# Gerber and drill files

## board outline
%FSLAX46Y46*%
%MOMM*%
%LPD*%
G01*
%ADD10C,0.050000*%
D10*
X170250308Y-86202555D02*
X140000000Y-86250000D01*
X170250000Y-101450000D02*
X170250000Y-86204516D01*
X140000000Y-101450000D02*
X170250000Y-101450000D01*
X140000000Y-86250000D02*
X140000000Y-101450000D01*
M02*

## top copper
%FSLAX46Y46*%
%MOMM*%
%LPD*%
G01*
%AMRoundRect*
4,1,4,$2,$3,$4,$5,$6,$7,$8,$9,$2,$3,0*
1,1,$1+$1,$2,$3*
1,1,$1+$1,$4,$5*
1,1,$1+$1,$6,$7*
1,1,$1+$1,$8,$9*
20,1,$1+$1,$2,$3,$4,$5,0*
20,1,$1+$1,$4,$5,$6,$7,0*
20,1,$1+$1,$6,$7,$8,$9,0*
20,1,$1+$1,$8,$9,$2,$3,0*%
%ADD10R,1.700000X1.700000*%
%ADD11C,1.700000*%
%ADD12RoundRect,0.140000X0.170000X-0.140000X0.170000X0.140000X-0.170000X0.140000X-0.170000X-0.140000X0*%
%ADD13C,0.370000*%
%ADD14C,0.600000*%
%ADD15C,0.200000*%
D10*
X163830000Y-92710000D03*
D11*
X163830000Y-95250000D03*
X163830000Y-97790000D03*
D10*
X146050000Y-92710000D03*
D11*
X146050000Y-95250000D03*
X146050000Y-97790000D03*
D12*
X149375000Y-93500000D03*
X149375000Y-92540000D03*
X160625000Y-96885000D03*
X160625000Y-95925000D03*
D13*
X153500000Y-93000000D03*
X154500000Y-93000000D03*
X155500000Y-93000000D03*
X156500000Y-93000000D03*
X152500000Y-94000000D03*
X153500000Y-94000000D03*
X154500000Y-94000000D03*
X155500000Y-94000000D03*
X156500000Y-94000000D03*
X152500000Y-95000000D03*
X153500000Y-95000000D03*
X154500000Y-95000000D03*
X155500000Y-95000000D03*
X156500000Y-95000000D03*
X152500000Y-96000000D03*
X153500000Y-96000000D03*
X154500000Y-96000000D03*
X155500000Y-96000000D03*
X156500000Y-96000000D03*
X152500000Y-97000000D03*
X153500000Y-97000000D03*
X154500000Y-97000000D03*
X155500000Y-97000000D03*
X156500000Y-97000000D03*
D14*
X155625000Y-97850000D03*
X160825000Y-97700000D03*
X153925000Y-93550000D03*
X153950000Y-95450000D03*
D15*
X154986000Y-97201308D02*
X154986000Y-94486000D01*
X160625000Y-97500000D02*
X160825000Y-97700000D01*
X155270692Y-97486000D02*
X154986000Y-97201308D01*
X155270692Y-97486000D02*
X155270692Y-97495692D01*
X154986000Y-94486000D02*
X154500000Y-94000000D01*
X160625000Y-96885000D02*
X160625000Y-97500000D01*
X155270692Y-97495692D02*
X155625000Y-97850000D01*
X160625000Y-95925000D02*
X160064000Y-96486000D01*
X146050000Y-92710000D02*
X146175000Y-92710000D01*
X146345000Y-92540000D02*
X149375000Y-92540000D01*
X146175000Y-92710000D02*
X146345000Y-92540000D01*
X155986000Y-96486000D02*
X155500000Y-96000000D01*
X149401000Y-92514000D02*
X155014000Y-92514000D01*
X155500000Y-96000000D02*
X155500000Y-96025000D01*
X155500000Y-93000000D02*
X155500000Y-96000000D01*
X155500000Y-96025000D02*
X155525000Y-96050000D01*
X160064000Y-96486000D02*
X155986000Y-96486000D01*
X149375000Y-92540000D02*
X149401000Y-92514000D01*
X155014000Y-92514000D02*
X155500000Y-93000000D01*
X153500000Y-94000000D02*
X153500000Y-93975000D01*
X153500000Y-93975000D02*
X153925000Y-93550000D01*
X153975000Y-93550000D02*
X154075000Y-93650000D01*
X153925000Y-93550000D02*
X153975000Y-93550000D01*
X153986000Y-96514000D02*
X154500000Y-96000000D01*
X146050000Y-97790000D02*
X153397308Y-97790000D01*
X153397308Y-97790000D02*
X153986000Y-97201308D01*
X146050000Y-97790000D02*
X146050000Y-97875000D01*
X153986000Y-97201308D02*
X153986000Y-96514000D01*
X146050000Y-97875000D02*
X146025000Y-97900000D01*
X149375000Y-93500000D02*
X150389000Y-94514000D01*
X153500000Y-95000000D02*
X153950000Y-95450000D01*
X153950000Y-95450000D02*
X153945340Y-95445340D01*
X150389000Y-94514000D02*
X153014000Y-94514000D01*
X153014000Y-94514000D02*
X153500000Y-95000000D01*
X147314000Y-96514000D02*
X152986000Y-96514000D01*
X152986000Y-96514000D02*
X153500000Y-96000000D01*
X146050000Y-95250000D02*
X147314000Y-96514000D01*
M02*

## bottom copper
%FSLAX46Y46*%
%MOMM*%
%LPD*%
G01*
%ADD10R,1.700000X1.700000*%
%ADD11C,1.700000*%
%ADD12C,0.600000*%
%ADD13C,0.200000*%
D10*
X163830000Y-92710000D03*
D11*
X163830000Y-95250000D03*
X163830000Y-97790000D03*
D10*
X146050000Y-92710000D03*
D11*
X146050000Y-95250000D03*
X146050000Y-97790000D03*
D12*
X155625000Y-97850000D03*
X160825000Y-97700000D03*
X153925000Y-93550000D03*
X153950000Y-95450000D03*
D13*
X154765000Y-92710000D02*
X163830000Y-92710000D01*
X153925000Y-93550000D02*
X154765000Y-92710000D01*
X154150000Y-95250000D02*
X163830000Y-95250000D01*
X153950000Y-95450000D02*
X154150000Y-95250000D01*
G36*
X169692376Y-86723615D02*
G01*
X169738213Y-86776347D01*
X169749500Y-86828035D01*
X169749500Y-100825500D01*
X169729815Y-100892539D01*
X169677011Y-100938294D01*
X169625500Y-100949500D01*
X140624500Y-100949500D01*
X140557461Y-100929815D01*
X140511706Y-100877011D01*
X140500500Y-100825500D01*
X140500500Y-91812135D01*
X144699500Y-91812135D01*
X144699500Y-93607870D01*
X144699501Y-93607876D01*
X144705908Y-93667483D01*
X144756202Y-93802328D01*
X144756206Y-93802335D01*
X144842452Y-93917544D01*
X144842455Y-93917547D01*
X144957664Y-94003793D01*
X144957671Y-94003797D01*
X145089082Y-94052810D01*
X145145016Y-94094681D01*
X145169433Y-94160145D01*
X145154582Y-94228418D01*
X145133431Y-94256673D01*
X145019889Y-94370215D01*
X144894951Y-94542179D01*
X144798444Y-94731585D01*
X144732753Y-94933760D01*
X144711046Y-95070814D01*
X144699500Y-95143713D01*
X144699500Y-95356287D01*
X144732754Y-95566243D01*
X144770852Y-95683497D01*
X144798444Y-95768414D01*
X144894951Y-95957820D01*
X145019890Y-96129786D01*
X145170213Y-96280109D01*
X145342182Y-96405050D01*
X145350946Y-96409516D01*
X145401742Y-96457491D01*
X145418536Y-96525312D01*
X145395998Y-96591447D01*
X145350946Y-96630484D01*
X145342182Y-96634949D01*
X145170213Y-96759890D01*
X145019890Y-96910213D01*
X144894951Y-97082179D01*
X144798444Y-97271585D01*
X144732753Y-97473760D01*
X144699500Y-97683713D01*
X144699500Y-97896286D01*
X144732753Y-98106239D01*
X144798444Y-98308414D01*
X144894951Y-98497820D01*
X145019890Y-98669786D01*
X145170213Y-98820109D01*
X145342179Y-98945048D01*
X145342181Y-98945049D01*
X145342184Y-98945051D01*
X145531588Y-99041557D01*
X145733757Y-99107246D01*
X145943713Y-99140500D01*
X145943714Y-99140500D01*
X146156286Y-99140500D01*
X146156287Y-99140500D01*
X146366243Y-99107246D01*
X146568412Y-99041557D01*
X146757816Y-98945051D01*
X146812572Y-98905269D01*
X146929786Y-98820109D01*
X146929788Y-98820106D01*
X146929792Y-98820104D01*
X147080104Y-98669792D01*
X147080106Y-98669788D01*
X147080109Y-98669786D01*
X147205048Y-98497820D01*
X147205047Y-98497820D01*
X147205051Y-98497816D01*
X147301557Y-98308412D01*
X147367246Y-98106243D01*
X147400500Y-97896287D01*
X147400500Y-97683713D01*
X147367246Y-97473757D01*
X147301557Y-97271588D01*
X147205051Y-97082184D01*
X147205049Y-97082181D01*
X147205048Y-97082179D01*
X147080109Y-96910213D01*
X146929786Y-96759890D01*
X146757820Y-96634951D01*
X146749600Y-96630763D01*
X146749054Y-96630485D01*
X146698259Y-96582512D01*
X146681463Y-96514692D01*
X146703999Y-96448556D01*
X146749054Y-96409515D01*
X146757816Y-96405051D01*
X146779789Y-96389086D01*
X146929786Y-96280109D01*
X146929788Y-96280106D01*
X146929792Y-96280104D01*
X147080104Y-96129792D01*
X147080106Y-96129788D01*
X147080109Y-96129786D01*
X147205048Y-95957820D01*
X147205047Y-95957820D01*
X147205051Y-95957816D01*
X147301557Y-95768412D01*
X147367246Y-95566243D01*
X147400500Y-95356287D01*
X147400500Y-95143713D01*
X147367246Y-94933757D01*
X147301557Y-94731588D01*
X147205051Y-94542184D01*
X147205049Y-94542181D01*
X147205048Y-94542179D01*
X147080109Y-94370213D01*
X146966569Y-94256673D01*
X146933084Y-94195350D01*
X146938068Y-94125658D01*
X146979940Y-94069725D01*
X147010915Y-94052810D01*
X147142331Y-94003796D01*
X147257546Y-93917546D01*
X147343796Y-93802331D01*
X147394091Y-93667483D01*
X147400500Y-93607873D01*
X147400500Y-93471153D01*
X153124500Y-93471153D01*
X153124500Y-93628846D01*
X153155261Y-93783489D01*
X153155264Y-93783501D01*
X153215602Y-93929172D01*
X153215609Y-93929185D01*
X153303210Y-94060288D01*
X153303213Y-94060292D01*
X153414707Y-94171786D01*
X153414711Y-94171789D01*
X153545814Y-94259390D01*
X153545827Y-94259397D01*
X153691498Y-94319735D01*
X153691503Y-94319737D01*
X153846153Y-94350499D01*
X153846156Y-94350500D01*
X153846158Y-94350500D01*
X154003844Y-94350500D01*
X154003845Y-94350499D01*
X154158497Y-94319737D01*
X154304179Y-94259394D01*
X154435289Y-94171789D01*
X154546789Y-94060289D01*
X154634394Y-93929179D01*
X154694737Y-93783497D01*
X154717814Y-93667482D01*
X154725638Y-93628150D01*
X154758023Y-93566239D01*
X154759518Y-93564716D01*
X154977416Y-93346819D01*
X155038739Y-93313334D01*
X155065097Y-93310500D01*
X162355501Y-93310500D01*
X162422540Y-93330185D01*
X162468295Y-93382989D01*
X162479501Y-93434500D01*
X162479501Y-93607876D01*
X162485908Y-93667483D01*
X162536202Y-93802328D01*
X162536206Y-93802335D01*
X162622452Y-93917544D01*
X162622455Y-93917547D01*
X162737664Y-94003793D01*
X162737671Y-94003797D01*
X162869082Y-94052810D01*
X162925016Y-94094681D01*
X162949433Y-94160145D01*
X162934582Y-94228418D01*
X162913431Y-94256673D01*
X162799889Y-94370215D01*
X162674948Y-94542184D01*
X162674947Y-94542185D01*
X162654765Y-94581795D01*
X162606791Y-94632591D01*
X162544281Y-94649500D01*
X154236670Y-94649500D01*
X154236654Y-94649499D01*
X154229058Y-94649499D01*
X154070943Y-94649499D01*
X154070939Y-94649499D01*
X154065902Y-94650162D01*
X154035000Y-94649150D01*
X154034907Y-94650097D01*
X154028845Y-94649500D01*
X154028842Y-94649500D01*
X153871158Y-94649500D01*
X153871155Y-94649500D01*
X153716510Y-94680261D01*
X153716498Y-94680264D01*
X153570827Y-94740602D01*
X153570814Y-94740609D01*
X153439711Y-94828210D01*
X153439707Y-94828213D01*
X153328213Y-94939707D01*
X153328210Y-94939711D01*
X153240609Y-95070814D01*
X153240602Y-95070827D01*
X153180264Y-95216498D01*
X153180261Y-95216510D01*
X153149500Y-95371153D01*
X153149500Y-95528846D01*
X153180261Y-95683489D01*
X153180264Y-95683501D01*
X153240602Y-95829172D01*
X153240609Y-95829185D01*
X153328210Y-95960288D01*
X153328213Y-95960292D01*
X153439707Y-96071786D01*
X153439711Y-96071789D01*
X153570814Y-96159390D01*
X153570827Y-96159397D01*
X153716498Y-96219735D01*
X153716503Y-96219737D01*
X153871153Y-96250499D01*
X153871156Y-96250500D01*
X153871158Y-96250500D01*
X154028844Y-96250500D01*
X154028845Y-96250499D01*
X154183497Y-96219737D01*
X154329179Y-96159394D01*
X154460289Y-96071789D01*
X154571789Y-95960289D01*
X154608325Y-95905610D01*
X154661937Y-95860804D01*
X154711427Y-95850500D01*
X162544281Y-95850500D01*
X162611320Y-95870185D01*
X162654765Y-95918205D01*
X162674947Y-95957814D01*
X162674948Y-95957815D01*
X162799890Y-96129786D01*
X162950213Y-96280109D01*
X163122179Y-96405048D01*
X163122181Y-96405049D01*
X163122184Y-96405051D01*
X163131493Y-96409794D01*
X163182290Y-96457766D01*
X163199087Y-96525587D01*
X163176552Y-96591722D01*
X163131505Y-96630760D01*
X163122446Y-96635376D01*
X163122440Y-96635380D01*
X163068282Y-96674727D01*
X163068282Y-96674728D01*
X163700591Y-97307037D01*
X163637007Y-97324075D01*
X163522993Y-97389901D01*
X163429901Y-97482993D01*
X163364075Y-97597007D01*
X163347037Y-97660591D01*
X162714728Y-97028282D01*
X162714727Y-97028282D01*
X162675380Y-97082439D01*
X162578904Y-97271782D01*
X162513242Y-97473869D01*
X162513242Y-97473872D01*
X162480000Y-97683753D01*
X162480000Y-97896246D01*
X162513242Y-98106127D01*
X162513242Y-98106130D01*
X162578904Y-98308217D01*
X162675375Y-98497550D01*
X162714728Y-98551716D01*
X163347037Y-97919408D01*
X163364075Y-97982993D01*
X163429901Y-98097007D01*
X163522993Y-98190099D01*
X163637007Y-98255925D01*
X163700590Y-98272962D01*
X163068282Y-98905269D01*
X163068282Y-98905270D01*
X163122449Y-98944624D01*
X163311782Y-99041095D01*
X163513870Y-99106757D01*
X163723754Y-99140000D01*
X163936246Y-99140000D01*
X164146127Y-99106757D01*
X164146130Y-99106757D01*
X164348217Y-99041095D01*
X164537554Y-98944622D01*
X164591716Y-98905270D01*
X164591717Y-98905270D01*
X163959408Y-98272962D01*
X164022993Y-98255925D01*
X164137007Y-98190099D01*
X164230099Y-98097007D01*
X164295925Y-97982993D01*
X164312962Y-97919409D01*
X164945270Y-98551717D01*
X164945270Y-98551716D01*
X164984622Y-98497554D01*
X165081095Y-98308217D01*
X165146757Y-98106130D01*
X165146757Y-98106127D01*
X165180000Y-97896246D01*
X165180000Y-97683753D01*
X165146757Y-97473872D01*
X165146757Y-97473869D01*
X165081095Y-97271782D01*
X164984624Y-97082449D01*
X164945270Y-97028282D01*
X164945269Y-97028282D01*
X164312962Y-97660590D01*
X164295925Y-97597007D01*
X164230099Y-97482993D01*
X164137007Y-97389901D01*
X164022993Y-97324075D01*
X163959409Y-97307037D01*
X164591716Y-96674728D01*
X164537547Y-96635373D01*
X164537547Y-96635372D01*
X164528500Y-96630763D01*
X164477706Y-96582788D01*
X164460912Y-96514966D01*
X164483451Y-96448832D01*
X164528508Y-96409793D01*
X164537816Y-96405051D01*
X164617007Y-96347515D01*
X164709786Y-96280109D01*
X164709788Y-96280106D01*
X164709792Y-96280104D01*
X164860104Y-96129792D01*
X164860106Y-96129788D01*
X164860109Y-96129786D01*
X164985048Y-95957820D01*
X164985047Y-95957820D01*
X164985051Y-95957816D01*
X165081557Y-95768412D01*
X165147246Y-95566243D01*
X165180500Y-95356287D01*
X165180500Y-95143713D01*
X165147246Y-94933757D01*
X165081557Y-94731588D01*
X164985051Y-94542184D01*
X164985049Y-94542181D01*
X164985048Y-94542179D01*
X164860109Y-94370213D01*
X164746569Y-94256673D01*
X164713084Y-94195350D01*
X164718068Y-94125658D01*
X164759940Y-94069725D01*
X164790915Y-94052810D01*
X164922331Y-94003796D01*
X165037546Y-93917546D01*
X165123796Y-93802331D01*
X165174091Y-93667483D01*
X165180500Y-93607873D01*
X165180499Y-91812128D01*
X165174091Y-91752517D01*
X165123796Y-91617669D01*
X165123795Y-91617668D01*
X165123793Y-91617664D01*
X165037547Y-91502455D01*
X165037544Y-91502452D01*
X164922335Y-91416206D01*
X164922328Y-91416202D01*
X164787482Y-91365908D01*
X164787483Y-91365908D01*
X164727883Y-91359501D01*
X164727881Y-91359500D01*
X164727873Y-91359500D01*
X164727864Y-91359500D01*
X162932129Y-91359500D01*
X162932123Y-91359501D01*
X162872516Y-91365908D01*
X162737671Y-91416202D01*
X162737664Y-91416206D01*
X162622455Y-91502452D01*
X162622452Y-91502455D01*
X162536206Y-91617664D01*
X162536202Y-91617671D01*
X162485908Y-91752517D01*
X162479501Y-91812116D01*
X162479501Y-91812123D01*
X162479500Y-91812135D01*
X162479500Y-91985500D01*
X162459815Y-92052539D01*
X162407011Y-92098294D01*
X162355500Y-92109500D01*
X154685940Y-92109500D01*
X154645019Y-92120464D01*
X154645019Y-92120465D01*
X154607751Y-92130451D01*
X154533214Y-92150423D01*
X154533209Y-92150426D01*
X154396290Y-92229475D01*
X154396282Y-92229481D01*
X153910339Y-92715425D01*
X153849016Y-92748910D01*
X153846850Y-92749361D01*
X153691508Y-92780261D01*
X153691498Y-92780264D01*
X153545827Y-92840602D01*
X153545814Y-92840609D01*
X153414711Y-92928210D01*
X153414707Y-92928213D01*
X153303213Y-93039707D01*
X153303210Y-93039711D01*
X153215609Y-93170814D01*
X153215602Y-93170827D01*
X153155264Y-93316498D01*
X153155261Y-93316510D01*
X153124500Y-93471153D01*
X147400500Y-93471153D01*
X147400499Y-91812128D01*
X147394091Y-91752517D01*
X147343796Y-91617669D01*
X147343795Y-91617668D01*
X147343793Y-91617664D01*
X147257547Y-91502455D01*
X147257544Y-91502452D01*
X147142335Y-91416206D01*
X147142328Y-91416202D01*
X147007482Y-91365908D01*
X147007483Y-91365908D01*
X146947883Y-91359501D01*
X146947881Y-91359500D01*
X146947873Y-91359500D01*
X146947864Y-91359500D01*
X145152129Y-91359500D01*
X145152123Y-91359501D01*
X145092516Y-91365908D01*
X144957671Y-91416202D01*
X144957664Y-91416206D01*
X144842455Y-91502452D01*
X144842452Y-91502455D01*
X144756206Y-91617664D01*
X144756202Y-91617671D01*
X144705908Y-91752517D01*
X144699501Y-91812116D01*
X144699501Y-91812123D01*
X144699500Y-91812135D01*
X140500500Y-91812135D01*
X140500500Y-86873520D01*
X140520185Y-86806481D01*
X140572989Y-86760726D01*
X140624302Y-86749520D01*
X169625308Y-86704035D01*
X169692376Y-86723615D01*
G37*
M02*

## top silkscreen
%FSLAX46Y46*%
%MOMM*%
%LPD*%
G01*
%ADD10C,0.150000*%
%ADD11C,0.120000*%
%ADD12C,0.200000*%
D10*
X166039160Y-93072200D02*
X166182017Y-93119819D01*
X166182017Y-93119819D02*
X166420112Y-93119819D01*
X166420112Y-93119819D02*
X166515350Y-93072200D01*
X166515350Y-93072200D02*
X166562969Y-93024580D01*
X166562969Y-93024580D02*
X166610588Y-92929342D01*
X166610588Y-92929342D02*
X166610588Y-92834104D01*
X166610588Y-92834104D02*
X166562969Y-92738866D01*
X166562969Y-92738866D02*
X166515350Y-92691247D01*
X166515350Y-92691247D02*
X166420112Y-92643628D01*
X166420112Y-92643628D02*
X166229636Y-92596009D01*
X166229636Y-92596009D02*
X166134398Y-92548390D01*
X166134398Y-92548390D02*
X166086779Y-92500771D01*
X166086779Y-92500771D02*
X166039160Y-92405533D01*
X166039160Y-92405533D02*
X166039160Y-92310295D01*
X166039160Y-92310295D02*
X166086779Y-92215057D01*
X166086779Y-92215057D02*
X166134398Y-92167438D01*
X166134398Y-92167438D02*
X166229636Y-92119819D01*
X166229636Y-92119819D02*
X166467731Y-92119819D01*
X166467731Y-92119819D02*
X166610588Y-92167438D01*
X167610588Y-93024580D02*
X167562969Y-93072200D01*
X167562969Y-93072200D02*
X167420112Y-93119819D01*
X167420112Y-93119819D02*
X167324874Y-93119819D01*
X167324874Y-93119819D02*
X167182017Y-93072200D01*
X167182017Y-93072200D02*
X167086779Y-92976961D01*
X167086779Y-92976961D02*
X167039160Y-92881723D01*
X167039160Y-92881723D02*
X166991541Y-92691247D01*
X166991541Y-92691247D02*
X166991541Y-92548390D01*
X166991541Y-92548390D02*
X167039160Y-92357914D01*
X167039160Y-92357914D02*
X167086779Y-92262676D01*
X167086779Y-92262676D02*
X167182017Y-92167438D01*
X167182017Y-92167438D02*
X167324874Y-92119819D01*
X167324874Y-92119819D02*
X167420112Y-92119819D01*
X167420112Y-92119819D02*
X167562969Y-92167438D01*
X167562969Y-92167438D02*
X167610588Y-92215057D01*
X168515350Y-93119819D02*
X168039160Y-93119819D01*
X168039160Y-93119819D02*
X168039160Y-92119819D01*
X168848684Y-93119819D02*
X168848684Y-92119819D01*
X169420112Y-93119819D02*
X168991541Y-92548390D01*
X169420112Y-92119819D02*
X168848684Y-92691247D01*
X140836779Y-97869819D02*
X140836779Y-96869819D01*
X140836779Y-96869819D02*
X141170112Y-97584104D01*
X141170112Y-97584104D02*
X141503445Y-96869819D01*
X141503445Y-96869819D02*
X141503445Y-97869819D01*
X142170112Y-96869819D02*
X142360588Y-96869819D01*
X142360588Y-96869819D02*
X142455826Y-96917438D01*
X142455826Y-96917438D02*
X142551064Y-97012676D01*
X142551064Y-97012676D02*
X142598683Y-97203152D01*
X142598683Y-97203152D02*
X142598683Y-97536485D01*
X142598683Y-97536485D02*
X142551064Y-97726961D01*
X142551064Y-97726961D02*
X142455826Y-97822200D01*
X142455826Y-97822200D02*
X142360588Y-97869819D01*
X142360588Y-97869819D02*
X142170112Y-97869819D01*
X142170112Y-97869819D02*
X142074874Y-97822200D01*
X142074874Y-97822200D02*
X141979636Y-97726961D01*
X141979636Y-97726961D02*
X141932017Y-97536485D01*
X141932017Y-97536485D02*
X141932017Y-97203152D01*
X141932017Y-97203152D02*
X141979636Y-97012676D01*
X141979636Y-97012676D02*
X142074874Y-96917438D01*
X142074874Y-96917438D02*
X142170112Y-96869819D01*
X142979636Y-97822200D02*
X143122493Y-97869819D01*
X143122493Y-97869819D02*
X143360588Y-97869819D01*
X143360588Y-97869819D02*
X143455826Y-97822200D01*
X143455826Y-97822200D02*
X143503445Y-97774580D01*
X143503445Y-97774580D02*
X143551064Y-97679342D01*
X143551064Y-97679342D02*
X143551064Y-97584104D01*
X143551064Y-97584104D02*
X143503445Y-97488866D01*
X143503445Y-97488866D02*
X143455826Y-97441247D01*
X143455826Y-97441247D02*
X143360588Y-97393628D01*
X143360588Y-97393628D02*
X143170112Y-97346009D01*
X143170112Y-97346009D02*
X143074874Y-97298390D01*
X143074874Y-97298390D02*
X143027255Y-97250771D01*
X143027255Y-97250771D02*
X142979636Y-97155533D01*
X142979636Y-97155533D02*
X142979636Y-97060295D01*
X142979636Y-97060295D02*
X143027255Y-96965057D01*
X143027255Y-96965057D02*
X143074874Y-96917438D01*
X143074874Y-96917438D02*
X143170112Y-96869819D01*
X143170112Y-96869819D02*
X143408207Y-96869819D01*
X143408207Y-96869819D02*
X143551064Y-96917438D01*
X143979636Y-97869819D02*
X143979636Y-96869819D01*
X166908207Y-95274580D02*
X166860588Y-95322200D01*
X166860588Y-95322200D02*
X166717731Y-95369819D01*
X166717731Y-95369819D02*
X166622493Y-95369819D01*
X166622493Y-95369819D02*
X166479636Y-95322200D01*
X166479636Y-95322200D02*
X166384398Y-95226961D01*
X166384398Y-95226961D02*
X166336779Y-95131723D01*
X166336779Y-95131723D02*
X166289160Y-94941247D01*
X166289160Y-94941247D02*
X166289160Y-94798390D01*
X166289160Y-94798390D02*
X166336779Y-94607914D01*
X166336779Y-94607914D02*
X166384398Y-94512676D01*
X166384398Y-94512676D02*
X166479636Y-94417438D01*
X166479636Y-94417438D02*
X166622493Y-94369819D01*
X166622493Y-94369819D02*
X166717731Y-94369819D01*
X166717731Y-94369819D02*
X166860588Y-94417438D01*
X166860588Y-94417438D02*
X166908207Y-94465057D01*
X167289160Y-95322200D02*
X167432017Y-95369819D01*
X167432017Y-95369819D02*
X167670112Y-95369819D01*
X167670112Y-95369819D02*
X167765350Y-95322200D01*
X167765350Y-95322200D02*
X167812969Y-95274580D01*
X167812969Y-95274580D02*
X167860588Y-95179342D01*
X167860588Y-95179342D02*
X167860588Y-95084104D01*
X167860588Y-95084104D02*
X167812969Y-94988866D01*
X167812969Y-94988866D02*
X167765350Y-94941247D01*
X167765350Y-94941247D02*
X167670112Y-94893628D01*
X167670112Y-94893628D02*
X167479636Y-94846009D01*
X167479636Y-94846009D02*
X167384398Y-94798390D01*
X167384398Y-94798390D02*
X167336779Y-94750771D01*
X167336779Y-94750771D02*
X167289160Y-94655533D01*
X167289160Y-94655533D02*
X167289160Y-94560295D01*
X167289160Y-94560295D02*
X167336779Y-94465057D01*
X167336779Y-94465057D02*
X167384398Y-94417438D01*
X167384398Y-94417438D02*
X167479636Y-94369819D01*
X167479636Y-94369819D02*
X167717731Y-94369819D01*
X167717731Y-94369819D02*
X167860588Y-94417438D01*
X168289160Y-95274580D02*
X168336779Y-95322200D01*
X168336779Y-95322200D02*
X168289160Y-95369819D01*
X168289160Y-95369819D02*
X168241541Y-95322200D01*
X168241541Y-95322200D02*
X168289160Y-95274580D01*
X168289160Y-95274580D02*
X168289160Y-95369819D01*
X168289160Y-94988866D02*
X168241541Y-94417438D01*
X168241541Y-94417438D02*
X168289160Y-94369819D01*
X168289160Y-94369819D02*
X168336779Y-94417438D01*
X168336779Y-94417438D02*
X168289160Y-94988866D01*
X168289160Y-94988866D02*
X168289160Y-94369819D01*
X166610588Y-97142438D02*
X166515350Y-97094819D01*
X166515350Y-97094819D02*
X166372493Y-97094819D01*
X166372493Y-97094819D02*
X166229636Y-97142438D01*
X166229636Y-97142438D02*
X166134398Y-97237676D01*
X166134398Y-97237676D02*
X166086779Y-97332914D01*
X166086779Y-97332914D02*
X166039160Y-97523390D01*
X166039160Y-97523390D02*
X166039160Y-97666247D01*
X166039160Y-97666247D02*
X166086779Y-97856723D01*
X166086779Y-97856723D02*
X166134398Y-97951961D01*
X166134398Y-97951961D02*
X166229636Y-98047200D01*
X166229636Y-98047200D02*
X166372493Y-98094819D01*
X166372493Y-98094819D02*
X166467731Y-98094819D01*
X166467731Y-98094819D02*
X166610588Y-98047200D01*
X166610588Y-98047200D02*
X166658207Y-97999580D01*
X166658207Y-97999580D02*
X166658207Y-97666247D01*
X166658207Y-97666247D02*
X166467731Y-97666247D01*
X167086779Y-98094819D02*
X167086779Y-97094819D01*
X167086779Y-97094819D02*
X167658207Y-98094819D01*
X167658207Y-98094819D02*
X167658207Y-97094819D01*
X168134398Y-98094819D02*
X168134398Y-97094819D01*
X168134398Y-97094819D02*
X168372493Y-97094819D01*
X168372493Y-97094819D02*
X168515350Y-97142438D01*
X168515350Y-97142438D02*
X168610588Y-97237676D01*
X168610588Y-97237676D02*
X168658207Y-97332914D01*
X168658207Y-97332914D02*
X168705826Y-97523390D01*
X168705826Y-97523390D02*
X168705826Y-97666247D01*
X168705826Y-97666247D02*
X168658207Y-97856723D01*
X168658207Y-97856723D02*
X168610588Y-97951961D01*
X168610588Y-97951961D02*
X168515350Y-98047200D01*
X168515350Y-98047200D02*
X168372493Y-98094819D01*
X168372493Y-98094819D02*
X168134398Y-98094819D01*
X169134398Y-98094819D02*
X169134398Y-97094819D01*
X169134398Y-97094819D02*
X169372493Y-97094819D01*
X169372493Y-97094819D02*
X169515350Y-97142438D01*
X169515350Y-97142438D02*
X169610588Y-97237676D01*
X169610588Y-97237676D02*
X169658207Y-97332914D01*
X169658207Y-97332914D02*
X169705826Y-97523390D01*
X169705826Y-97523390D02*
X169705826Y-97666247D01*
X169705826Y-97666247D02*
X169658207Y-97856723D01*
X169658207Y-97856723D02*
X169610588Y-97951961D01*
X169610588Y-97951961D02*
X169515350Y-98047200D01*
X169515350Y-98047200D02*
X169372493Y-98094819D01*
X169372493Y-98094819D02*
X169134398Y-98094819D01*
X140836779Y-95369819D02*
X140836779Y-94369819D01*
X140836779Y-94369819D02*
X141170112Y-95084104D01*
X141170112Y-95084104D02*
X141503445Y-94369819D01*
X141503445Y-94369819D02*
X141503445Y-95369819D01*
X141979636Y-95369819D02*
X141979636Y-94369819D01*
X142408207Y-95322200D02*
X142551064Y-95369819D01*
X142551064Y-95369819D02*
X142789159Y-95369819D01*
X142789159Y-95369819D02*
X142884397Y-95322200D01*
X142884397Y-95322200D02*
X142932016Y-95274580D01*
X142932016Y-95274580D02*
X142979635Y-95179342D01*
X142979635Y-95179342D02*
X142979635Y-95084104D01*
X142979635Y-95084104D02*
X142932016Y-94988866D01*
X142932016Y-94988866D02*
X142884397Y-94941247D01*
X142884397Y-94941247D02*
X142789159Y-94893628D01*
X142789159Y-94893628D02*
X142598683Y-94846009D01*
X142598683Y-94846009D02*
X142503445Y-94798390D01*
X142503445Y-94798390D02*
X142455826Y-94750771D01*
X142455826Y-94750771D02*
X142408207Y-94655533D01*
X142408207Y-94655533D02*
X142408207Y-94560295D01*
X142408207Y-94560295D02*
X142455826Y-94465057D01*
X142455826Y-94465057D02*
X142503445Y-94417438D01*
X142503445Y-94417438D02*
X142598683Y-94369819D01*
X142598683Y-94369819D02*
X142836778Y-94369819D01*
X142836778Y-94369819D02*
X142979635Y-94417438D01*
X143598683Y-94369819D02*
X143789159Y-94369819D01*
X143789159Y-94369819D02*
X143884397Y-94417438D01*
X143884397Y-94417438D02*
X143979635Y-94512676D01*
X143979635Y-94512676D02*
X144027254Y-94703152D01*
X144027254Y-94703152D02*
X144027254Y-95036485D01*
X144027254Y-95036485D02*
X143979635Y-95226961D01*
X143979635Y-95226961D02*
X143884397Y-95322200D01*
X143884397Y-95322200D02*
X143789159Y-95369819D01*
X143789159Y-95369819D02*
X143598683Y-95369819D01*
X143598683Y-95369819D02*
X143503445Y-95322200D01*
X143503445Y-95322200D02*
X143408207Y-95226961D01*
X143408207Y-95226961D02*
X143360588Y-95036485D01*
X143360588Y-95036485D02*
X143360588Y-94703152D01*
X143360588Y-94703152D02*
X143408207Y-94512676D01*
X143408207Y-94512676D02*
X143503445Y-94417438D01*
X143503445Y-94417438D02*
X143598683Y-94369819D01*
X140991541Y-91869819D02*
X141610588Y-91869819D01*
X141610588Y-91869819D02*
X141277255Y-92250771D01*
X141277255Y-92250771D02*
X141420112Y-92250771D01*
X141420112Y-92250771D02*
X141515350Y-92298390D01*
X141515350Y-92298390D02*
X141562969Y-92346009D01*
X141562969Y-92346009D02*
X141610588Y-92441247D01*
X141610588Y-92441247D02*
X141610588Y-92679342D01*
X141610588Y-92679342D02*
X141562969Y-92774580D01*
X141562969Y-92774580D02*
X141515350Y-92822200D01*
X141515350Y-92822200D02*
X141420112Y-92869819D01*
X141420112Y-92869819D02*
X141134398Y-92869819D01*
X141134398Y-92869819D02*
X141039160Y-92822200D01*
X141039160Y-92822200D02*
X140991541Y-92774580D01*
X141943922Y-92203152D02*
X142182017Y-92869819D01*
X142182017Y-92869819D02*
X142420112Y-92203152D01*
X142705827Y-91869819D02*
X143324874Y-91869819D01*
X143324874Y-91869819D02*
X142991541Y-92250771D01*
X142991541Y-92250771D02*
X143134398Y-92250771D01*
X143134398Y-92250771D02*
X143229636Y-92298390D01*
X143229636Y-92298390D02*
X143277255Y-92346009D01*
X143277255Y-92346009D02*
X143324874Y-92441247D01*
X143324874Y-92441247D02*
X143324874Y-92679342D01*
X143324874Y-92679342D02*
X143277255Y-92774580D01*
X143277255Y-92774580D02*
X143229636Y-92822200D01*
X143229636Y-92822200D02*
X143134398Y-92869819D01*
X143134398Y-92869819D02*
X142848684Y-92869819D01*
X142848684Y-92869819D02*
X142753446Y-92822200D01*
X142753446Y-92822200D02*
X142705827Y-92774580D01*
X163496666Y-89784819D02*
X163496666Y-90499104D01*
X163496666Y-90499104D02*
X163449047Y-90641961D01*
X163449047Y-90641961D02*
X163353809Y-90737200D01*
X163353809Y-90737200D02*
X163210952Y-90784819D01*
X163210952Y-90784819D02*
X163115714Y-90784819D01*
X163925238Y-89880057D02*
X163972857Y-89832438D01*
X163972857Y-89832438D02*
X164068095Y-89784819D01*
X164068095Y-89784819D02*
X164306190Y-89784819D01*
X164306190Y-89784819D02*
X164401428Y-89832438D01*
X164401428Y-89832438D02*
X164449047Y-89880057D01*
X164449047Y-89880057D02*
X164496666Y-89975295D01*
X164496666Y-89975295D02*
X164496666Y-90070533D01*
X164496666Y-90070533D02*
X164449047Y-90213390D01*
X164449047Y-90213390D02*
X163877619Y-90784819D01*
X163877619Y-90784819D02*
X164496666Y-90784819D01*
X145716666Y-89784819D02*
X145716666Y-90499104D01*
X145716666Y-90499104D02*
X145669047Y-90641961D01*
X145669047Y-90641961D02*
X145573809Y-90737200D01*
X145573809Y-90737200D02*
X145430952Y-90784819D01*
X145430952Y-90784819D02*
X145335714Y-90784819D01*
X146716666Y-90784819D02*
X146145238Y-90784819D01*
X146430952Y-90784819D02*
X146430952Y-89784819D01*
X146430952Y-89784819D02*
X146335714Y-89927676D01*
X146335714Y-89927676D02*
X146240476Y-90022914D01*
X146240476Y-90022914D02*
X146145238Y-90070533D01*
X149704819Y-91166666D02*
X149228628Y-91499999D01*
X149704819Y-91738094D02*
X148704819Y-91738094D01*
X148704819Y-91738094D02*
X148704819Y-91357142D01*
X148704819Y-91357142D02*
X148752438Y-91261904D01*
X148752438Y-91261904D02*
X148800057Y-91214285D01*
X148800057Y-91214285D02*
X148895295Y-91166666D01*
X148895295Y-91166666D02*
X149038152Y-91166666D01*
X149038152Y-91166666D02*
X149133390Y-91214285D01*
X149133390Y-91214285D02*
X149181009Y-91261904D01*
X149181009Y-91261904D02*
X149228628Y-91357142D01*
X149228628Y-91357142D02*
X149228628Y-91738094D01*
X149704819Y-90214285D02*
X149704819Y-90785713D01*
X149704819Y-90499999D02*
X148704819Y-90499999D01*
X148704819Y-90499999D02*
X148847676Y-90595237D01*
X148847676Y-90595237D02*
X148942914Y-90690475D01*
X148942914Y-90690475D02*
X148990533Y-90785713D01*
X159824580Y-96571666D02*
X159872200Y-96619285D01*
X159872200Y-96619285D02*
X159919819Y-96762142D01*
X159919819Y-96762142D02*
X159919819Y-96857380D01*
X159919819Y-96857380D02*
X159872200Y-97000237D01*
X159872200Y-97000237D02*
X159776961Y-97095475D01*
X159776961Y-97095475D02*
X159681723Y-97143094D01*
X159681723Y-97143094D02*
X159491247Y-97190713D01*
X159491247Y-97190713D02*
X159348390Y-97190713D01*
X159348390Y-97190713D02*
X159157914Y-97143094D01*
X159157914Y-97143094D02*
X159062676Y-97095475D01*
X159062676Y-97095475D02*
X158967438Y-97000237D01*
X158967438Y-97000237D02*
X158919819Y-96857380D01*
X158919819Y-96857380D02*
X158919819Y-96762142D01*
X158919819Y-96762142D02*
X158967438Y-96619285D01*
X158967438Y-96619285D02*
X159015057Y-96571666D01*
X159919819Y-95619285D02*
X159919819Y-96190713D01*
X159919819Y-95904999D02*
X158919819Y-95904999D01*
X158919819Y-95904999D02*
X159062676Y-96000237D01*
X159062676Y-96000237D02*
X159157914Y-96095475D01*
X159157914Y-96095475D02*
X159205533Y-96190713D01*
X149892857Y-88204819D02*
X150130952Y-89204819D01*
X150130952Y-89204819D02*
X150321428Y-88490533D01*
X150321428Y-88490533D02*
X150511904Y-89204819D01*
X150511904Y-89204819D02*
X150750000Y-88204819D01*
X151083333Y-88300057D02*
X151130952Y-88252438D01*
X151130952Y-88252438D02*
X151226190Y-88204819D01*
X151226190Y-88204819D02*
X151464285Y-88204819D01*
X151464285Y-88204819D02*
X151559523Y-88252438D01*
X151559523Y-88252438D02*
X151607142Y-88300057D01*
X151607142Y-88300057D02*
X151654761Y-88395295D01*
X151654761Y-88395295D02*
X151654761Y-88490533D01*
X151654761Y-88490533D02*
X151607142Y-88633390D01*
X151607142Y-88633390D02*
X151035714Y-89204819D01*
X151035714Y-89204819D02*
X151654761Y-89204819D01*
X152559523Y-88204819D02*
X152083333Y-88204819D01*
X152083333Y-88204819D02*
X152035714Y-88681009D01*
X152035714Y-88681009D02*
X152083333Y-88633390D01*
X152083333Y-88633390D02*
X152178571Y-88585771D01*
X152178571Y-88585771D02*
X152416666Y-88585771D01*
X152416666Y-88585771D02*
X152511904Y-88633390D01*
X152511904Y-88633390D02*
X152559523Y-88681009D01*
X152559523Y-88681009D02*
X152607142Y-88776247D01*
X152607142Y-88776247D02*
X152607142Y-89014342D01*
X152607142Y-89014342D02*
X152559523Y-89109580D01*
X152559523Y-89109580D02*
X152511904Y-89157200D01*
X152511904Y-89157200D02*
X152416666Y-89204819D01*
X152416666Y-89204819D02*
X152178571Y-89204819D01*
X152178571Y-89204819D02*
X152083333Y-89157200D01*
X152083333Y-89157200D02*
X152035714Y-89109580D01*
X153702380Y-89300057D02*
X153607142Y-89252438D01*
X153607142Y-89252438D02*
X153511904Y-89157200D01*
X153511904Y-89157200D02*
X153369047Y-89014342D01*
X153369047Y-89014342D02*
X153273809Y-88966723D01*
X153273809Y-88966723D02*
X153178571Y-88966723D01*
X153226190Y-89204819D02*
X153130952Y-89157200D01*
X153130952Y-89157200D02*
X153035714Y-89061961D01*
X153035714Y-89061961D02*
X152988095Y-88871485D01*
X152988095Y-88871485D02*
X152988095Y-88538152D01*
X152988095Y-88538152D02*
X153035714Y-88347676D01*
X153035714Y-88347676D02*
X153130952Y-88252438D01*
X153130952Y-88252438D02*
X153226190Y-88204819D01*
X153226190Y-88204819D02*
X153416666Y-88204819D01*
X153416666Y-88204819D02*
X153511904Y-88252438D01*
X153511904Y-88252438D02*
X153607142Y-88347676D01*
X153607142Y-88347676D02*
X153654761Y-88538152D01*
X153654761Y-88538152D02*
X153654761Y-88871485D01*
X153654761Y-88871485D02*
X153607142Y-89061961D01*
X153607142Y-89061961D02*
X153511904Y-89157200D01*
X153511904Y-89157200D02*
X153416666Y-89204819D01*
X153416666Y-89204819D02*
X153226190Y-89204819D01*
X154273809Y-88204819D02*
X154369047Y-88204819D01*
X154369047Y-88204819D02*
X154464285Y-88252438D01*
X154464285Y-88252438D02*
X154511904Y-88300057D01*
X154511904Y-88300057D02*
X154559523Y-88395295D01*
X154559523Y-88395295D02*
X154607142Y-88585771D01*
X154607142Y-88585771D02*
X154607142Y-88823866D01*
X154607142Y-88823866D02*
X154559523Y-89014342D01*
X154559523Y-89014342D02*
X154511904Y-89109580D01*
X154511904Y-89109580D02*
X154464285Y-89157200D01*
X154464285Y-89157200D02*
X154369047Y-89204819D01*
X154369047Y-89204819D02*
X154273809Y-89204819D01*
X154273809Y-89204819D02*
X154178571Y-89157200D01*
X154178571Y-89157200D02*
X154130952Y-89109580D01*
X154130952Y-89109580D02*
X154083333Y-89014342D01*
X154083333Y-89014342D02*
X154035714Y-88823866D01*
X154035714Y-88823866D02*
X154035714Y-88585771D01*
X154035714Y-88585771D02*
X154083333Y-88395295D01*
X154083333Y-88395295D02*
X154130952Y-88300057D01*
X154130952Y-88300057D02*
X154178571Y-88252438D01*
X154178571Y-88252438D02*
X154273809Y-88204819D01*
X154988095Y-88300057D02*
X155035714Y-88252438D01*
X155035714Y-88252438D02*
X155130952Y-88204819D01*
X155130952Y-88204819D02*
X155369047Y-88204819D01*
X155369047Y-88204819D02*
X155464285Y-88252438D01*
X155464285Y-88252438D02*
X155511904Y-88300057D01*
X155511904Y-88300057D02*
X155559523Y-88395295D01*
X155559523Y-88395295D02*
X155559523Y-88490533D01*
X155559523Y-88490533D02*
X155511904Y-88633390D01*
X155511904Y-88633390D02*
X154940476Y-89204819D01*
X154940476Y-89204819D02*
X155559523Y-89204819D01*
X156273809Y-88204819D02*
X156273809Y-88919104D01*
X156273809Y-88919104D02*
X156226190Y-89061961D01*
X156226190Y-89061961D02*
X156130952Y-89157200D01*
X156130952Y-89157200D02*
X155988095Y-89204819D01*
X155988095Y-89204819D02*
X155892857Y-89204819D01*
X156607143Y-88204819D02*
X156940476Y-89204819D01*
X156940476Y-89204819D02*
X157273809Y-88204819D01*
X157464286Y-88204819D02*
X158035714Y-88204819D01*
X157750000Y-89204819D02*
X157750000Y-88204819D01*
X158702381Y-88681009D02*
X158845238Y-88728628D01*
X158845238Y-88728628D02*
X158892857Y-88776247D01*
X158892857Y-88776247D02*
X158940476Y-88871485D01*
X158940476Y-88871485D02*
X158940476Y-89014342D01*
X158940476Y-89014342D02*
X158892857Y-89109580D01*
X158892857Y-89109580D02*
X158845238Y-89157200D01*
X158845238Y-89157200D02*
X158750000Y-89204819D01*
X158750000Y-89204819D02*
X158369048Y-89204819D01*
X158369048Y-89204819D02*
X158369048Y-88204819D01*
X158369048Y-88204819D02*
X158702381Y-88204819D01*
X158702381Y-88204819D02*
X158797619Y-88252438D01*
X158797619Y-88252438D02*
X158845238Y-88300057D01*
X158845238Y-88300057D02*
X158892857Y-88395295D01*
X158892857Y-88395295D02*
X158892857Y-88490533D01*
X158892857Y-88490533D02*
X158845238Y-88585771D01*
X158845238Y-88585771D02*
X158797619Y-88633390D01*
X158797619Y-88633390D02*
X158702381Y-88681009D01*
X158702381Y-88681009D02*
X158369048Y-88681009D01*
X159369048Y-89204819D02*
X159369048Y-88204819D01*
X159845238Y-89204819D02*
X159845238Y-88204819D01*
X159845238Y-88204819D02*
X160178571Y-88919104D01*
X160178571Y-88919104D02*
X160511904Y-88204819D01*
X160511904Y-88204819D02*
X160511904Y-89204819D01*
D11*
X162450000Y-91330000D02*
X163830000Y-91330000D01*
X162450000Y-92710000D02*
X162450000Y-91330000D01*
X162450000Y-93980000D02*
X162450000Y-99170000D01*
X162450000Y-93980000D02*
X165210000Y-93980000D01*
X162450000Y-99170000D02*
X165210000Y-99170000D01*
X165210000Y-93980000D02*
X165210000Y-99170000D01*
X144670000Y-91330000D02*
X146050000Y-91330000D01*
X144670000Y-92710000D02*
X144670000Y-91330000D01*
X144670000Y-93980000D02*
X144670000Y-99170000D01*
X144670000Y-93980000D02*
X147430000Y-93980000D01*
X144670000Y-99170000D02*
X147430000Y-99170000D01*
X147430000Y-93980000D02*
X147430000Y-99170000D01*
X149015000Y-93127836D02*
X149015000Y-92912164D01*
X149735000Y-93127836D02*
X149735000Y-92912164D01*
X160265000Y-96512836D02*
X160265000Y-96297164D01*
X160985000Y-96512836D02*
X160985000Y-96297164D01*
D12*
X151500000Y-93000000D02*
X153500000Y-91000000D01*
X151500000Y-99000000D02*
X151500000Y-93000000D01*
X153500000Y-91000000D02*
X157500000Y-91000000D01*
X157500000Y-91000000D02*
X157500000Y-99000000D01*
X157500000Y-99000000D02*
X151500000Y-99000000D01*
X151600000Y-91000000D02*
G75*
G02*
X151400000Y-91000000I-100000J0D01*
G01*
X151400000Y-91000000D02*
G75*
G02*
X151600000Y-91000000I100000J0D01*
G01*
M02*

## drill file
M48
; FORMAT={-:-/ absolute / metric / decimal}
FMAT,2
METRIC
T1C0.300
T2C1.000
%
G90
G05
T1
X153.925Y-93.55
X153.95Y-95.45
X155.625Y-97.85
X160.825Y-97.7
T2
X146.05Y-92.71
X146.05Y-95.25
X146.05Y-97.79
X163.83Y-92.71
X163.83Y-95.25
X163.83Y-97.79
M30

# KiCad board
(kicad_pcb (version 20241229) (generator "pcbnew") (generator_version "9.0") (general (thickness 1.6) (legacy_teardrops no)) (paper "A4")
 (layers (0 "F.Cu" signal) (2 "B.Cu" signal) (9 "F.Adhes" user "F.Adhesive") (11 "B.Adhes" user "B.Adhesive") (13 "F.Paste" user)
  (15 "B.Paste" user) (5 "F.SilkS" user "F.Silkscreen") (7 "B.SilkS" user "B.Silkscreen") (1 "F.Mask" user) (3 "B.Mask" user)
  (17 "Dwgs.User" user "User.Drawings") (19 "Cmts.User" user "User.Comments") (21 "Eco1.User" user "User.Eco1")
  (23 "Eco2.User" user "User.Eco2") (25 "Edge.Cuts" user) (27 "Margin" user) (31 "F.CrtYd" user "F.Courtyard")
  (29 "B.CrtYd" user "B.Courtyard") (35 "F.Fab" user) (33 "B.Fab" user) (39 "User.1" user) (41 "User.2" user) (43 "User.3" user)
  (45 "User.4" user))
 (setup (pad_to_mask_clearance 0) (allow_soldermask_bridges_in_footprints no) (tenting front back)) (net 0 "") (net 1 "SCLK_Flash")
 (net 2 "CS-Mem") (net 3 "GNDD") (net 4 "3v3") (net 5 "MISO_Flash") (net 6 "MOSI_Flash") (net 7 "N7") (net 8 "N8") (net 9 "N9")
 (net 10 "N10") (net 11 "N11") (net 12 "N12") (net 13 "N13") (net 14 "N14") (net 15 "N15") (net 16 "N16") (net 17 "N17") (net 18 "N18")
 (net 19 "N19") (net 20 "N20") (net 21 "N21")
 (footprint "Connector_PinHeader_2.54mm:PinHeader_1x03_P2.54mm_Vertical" (layer "F.Cu") (at 163.83 92.71)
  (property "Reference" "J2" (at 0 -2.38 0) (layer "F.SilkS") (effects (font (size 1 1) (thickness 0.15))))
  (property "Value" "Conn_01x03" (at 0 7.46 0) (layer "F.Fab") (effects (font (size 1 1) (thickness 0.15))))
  (fp_line (start -1.38 -1.38) (end 0 -1.38) (stroke (width 0.12) (type solid)) (layer "F.SilkS"))
  (fp_line (start -1.38 0) (end -1.38 -1.38) (stroke (width 0.12) (type solid)) (layer "F.SilkS"))
  (fp_line (start -1.38 1.27) (end -1.38 6.46) (stroke (width 0.12) (type solid)) (layer "F.SilkS"))
  (fp_line (start -1.38 1.27) (end 1.38 1.27) (stroke (width 0.12) (type solid)) (layer "F.SilkS"))
  (fp_line (start -1.38 6.46) (end 1.38 6.46) (stroke (width 0.12) (type solid)) (layer "F.SilkS"))
  (fp_line (start 1.38 1.27) (end 1.38 6.46) (stroke (width 0.12) (type solid)) (layer "F.SilkS"))
  (pad "1" thru_hole rect (at 0 0) (size 1.7 1.7) (drill 1) (layers "*.Cu" "*.Mask") (remove_unused_layers no) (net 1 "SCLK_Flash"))
  (pad "2" thru_hole circle (at 0 2.54) (size 1.7 1.7) (drill 1) (layers "*.Cu" "*.Mask") (remove_unused_layers no) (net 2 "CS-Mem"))
  (pad "3" thru_hole circle (at 0 5.08) (size 1.7 1.7) (drill 1) (layers "*.Cu" "*.Mask") (remove_unused_layers no) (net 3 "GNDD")))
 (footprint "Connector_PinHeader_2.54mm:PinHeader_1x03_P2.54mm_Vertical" (layer "F.Cu") (at 146.05 92.71)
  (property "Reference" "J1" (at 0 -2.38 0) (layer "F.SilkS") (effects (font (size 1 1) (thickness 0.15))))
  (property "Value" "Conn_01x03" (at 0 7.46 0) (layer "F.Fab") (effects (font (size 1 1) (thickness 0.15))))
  (fp_line (start -1.38 -1.38) (end 0 -1.38) (stroke (width 0.12) (type solid)) (layer "F.SilkS"))
  (fp_line (start -1.38 0) (end -1.38 -1.38) (stroke (width 0.12) (type solid)) (layer "F.SilkS"))
  (fp_line (start -1.38 1.27) (end -1.38 6.46) (stroke (width 0.12) (type solid)) (layer "F.SilkS"))
  (fp_line (start -1.38 1.27) (end 1.38 1.27) (stroke (width 0.12) (type solid)) (layer "F.SilkS"))
  (fp_line (start -1.38 6.46) (end 1.38 6.46) (stroke (width 0.12) (type solid)) (layer "F.SilkS"))
  (fp_line (start 1.38 1.27) (end 1.38 6.46) (stroke (width 0.12) (type solid)) (layer "F.SilkS"))
  (pad "1" thru_hole rect (at 0 0) (size 1.7 1.7) (drill 1) (layers "*.Cu" "*.Mask") (remove_unused_layers no) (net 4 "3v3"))
  (pad "2" thru_hole circle (at 0 2.54) (size 1.7 1.7) (drill 1) (layers "*.Cu" "*.Mask") (remove_unused_layers no) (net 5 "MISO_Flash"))
  (pad "3" thru_hole circle (at 0 5.08) (size 1.7 1.7) (drill 1) (layers "*.Cu" "*.Mask") (remove_unused_layers no) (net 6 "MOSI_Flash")))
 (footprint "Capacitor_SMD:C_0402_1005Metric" (layer "F.Cu") (at 149.375 93.02 90)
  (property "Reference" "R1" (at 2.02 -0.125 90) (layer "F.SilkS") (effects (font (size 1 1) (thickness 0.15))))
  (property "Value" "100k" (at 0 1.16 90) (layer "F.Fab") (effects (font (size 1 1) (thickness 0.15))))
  (fp_line (start -0.107836 -0.36) (end 0.107836 -0.36) (stroke (width 0.12) (type solid)) (layer "F.SilkS"))
  (fp_line (start -0.107836 0.36) (end 0.107836 0.36) (stroke (width 0.12) (type solid)) (layer "F.SilkS"))
  (pad "1" smd roundrect (at -0.48 0 90) (size 0.56 0.62) (layers "F.Cu" "F.Mask" "F.Paste") (roundrect_rratio 0.25) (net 2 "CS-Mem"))
  (pad "2" smd roundrect (at 0.48 0 90) (size 0.56 0.62) (layers "F.Cu" "F.Mask" "F.Paste") (roundrect_rratio 0.25) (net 4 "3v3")))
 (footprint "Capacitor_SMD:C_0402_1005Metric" (layer "F.Cu") (at 160.625 96.405 90)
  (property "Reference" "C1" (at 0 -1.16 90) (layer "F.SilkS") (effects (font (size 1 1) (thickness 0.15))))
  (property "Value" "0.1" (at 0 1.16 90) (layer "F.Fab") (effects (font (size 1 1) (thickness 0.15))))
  (fp_line (start -0.107836 -0.36) (end 0.107836 -0.36) (stroke (width 0.12) (type solid)) (layer "F.SilkS"))
  (fp_line (start -0.107836 0.36) (end 0.107836 0.36) (stroke (width 0.12) (type solid)) (layer "F.SilkS"))
  (pad "1" smd roundrect (at -0.48 0 90) (size 0.56 0.62) (layers "F.Cu" "F.Mask" "F.Paste") (roundrect_rratio 0.25) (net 3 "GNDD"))
  (pad "2" smd roundrect (at 0.48 0 90) (size 0.56 0.62) (layers "F.Cu" "F.Mask" "F.Paste") (roundrect_rratio 0.25) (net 4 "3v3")))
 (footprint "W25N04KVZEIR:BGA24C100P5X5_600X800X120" (layer "F.Cu") (at 154.5 95)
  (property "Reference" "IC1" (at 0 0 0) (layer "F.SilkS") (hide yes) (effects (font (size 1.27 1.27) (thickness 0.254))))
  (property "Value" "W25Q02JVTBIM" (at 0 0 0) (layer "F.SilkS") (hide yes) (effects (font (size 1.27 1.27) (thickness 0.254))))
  (fp_line (start -3 -2) (end -1 -4) (stroke (width 0.2) (type solid)) (layer "F.SilkS"))
  (fp_line (start -3 4) (end -3 -2) (stroke (width 0.2) (type solid)) (layer "F.SilkS"))
  (fp_line (start -1 -4) (end 3 -4) (stroke (width 0.2) (type solid)) (layer "F.SilkS"))
  (fp_line (start 3 -4) (end 3 4) (stroke (width 0.2) (type solid)) (layer "F.SilkS"))
  (fp_line (start 3 4) (end -3 4) (stroke (width 0.2) (type solid)) (layer "F.SilkS"))
  (fp_circle (center -3 -4) (end -3 -3.9) (stroke (width 0.2) (type solid)) (fill no) (layer "F.SilkS"))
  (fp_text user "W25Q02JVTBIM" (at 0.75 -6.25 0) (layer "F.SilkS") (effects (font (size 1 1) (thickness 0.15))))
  (pad "A2" smd circle (at -1 -2 90) (size 0.37 0.37) (layers "F.Cu" "F.Mask" "F.Paste") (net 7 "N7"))
  (pad "A3" smd circle (at 0 -2 90) (size 0.37 0.37) (layers "F.Cu" "F.Mask" "F.Paste") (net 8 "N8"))
  (pad "A4" smd circle (at 1 -2 90) (size 0.37 0.37) (layers "F.Cu" "F.Mask" "F.Paste") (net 4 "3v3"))
  (pad "A5" smd circle (at 2 -2 90) (size 0.37 0.37) (layers "F.Cu" "F.Mask" "F.Paste") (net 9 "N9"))
  (pad "B1" smd circle (at -2 -1 90) (size 0.37 0.37) (layers "F.Cu" "F.Mask" "F.Paste") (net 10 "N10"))
  (pad "B2" smd circle (at -1 -1 90) (size 0.37 0.37) (layers "F.Cu" "F.Mask" "F.Paste") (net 1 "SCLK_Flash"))
  (pad "B3" smd circle (at 0 -1 90) (size 0.37 0.37) (layers "F.Cu" "F.Mask" "F.Paste") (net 3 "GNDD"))
  (pad "B4" smd circle (at 1 -1 90) (size 0.37 0.37) (layers "F.Cu" "F.Mask" "F.Paste") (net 4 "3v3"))
  (pad "B5" smd circle (at 2 -1 90) (size 0.37 0.37) (layers "F.Cu" "F.Mask" "F.Paste") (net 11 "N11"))
  (pad "C1" smd circle (at -2 0 90) (size 0.37 0.37) (layers "F.Cu" "F.Mask" "F.Paste") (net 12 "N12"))
  (pad "C2" smd circle (at -1 0 90) (size 0.37 0.37) (layers "F.Cu" "F.Mask" "F.Paste") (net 2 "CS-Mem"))
  (pad "C3" smd circle (at 0 0 90) (size 0.37 0.37) (layers "F.Cu" "F.Mask" "F.Paste") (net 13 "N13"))
  (pad "C4" smd circle (at 1 0 90) (size 0.37 0.37) (layers "F.Cu" "F.Mask" "F.Paste") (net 4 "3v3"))
  (pad "C5" smd circle (at 2 0 90) (size 0.37 0.37) (layers "F.Cu" "F.Mask" "F.Paste") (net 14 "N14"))
  (pad "D1" smd circle (at -2 1 90) (size 0.37 0.37) (layers "F.Cu" "F.Mask" "F.Paste") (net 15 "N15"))
  (pad "D2" smd circle (at -1 1 90) (size 0.37 0.37) (layers "F.Cu" "F.Mask" "F.Paste") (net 5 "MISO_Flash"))
  (pad "D3" smd circle (at 0 1 90) (size 0.37 0.37) (layers "F.Cu" "F.Mask" "F.Paste") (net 6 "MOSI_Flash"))
  (pad "D4" smd circle (at 1 1 90) (size 0.37 0.37) (layers "F.Cu" "F.Mask" "F.Paste") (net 4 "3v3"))
  (pad "D5" smd circle (at 2 1 90) (size 0.37 0.37) (layers "F.Cu" "F.Mask" "F.Paste") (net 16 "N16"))
  (pad "E1" smd circle (at -2 2 90) (size 0.37 0.37) (layers "F.Cu" "F.Mask" "F.Paste") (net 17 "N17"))
  (pad "E2" smd circle (at -1 2 90) (size 0.37 0.37) (layers "F.Cu" "F.Mask" "F.Paste") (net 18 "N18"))
  (pad "E3" smd circle (at 0 2 90) (size 0.37 0.37) (layers "F.Cu" "F.Mask" "F.Paste") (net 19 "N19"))
  (pad "E4" smd circle (at 1 2 90) (size 0.37 0.37) (layers "F.Cu" "F.Mask" "F.Paste") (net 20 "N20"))
  (pad "E5" smd circle (at 2 2 90) (size 0.37 0.37) (layers "F.Cu" "F.Mask" "F.Paste") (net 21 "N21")))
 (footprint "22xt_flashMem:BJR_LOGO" (layer "B.Cu") (at 167.75 89 180)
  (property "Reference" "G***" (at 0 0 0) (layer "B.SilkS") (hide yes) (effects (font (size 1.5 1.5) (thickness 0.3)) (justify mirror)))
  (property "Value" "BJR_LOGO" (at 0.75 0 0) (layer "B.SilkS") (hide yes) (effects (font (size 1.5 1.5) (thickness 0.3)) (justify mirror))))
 (gr_line (start 170.250308 86.202555) (end 140 86.25) (stroke (width 0.05) (type default)) (layer "Edge.Cuts"))
 (gr_line (start 170.25 101.45) (end 170.25 86.204516) (stroke (width 0.05) (type default)) (layer "Edge.Cuts"))
 (gr_line (start 140 101.45) (end 170.25 101.45) (stroke (width 0.05) (type default)) (layer "Edge.Cuts"))
 (gr_line (start 140 86.25) (end 140 101.45) (stroke (width 0.05) (type default)) (layer "Edge.Cuts"))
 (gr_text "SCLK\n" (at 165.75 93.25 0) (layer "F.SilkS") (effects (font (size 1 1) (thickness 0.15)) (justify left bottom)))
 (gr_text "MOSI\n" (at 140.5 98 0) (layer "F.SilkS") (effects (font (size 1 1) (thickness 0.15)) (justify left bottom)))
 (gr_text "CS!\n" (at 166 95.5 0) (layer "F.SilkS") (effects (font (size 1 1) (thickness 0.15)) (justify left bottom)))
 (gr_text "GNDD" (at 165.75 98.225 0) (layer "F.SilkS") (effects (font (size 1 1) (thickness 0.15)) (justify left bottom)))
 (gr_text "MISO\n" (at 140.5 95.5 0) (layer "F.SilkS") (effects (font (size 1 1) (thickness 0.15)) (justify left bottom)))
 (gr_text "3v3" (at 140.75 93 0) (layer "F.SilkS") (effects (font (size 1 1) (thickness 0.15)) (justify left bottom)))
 (segment (start 154.986 97.201308) (end 154.986 94.486) (width 0.2) (layer "F.Cu") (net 3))
 (segment (start 160.625 97.5) (end 160.825 97.7) (width 0.2) (layer "F.Cu") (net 3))
 (segment (start 155.270692 97.486) (end 154.986 97.201308) (width 0.2) (layer "F.Cu") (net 3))
 (segment (start 155.270692 97.486) (end 155.270692 97.495692) (width 0.2) (layer "F.Cu") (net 3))
 (segment (start 154.986 94.486) (end 154.5 94) (width 0.2) (layer "F.Cu") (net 3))
 (segment (start 160.625 96.885) (end 160.625 97.5) (width 0.2) (layer "F.Cu") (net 3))
 (segment (start 155.270692 97.495692) (end 155.625 97.85) (width 0.2) (layer "F.Cu") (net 3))
 (via (at 155.625 97.85) (size 0.6) (drill 0.3) (layers "F.Cu" "B.Cu") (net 3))
 (via (at 160.825 97.7) (size 0.6) (drill 0.3) (layers "F.Cu" "B.Cu") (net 3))
 (segment (start 160.625 95.925) (end 160.064 96.486) (width 0.2) (layer "F.Cu") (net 4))
 (segment (start 146.05 92.71) (end 146.175 92.71) (width 0.2) (layer "F.Cu") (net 4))
 (segment (start 146.345 92.54) (end 149.375 92.54) (width 0.2) (layer "F.Cu") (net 4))
 (segment (start 146.175 92.71) (end 146.345 92.54) (width 0.2) (layer "F.Cu") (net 4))
 (segment (start 155.986 96.486) (end 155.5 96) (width 0.2) (layer "F.Cu") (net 4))
 (segment (start 149.401 92.514) (end 155.014 92.514) (width 0.2) (layer "F.Cu") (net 4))
 (segment (start 155.5 96) (end 155.5 96.025) (width 0.2) (layer "F.Cu") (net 4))
 (segment (start 155.5 93) (end 155.5 96) (width 0.2) (layer "F.Cu") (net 4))
 (segment (start 155.5 96.025) (end 155.525 96.05) (width 0.2) (layer "F.Cu") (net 4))
 (segment (start 160.064 96.486) (end 155.986 96.486) (width 0.2) (layer "F.Cu") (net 4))
 (segment (start 149.375 92.54) (end 149.401 92.514) (width 0.2) (layer "F.Cu") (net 4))
 (segment (start 155.014 92.514) (end 155.5 93) (width 0.2) (layer "F.Cu") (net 4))
 (segment (start 153.5 94) (end 153.5 93.975) (width 0.2) (layer "F.Cu") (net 1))
 (segment (start 153.5 93.975) (end 153.925 93.55) (width 0.2) (layer "F.Cu") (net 1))
 (segment (start 153.975 93.55) (end 154.075 93.65) (width 0.2) (layer "F.Cu") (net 1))
 (segment (start 153.925 93.55) (end 153.975 93.55) (width 0.2) (layer "F.Cu") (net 1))
 (via (at 153.925 93.55) (size 0.6) (drill 0.3) (layers "F.Cu" "B.Cu") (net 1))
 (segment (start 154.765 92.71) (end 163.83 92.71) (width 0.2) (layer "B.Cu") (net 1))
 (segment (start 153.925 93.55) (end 154.765 92.71) (width 0.2) (layer "B.Cu") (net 1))
 (segment (start 153.986 96.514) (end 154.5 96) (width 0.2) (layer "F.Cu") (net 6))
 (segment (start 146.05 97.79) (end 153.397308 97.79) (width 0.2) (layer "F.Cu") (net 6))
 (segment (start 153.397308 97.79) (end 153.986 97.201308) (width 0.2) (layer "F.Cu") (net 6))
 (segment (start 146.05 97.79) (end 146.05 97.875) (width 0.2) (layer "F.Cu") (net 6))
 (segment (start 153.986 97.201308) (end 153.986 96.514) (width 0.2) (layer "F.Cu") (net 6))
 (segment (start 146.05 97.875) (end 146.025 97.9) (width 0.2) (layer "F.Cu") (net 6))
 (segment (start 149.375 93.5) (end 150.389 94.514) (width 0.2) (layer "F.Cu") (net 2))
 (segment (start 153.5 95) (end 153.95 95.45) (width 0.2) (layer "F.Cu") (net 2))
 (segment (start 153.95 95.45) (end 153.94534 95.44534) (width 0.2) (layer "F.Cu") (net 2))
 (segment (start 150.389 94.514) (end 153.014 94.514) (width 0.2) (layer "F.Cu") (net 2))
 (segment (start 153.014 94.514) (end 153.5 95) (width 0.2) (layer "F.Cu") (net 2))
 (via (at 153.95 95.45) (size 0.6) (drill 0.3) (layers "F.Cu" "B.Cu") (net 2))
 (segment (start 154.15 95.25) (end 163.83 95.25) (width 0.2) (layer "B.Cu") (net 2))
 (segment (start 153.95 95.45) (end 154.15 95.25) (width 0.2) (layer "B.Cu") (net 2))
 (segment (start 147.314 96.514) (end 152.986 96.514) (width 0.2) (layer "F.Cu") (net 5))
 (segment (start 152.986 96.514) (end 153.5 96) (width 0.2) (layer "F.Cu") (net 5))
 (segment (start 146.05 95.25) (end 147.314 96.514) (width 0.2) (layer "F.Cu") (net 5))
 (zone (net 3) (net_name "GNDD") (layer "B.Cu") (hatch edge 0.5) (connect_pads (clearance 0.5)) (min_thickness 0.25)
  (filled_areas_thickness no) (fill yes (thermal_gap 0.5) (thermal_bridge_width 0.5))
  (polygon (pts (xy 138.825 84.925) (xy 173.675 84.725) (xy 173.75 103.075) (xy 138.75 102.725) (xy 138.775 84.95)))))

